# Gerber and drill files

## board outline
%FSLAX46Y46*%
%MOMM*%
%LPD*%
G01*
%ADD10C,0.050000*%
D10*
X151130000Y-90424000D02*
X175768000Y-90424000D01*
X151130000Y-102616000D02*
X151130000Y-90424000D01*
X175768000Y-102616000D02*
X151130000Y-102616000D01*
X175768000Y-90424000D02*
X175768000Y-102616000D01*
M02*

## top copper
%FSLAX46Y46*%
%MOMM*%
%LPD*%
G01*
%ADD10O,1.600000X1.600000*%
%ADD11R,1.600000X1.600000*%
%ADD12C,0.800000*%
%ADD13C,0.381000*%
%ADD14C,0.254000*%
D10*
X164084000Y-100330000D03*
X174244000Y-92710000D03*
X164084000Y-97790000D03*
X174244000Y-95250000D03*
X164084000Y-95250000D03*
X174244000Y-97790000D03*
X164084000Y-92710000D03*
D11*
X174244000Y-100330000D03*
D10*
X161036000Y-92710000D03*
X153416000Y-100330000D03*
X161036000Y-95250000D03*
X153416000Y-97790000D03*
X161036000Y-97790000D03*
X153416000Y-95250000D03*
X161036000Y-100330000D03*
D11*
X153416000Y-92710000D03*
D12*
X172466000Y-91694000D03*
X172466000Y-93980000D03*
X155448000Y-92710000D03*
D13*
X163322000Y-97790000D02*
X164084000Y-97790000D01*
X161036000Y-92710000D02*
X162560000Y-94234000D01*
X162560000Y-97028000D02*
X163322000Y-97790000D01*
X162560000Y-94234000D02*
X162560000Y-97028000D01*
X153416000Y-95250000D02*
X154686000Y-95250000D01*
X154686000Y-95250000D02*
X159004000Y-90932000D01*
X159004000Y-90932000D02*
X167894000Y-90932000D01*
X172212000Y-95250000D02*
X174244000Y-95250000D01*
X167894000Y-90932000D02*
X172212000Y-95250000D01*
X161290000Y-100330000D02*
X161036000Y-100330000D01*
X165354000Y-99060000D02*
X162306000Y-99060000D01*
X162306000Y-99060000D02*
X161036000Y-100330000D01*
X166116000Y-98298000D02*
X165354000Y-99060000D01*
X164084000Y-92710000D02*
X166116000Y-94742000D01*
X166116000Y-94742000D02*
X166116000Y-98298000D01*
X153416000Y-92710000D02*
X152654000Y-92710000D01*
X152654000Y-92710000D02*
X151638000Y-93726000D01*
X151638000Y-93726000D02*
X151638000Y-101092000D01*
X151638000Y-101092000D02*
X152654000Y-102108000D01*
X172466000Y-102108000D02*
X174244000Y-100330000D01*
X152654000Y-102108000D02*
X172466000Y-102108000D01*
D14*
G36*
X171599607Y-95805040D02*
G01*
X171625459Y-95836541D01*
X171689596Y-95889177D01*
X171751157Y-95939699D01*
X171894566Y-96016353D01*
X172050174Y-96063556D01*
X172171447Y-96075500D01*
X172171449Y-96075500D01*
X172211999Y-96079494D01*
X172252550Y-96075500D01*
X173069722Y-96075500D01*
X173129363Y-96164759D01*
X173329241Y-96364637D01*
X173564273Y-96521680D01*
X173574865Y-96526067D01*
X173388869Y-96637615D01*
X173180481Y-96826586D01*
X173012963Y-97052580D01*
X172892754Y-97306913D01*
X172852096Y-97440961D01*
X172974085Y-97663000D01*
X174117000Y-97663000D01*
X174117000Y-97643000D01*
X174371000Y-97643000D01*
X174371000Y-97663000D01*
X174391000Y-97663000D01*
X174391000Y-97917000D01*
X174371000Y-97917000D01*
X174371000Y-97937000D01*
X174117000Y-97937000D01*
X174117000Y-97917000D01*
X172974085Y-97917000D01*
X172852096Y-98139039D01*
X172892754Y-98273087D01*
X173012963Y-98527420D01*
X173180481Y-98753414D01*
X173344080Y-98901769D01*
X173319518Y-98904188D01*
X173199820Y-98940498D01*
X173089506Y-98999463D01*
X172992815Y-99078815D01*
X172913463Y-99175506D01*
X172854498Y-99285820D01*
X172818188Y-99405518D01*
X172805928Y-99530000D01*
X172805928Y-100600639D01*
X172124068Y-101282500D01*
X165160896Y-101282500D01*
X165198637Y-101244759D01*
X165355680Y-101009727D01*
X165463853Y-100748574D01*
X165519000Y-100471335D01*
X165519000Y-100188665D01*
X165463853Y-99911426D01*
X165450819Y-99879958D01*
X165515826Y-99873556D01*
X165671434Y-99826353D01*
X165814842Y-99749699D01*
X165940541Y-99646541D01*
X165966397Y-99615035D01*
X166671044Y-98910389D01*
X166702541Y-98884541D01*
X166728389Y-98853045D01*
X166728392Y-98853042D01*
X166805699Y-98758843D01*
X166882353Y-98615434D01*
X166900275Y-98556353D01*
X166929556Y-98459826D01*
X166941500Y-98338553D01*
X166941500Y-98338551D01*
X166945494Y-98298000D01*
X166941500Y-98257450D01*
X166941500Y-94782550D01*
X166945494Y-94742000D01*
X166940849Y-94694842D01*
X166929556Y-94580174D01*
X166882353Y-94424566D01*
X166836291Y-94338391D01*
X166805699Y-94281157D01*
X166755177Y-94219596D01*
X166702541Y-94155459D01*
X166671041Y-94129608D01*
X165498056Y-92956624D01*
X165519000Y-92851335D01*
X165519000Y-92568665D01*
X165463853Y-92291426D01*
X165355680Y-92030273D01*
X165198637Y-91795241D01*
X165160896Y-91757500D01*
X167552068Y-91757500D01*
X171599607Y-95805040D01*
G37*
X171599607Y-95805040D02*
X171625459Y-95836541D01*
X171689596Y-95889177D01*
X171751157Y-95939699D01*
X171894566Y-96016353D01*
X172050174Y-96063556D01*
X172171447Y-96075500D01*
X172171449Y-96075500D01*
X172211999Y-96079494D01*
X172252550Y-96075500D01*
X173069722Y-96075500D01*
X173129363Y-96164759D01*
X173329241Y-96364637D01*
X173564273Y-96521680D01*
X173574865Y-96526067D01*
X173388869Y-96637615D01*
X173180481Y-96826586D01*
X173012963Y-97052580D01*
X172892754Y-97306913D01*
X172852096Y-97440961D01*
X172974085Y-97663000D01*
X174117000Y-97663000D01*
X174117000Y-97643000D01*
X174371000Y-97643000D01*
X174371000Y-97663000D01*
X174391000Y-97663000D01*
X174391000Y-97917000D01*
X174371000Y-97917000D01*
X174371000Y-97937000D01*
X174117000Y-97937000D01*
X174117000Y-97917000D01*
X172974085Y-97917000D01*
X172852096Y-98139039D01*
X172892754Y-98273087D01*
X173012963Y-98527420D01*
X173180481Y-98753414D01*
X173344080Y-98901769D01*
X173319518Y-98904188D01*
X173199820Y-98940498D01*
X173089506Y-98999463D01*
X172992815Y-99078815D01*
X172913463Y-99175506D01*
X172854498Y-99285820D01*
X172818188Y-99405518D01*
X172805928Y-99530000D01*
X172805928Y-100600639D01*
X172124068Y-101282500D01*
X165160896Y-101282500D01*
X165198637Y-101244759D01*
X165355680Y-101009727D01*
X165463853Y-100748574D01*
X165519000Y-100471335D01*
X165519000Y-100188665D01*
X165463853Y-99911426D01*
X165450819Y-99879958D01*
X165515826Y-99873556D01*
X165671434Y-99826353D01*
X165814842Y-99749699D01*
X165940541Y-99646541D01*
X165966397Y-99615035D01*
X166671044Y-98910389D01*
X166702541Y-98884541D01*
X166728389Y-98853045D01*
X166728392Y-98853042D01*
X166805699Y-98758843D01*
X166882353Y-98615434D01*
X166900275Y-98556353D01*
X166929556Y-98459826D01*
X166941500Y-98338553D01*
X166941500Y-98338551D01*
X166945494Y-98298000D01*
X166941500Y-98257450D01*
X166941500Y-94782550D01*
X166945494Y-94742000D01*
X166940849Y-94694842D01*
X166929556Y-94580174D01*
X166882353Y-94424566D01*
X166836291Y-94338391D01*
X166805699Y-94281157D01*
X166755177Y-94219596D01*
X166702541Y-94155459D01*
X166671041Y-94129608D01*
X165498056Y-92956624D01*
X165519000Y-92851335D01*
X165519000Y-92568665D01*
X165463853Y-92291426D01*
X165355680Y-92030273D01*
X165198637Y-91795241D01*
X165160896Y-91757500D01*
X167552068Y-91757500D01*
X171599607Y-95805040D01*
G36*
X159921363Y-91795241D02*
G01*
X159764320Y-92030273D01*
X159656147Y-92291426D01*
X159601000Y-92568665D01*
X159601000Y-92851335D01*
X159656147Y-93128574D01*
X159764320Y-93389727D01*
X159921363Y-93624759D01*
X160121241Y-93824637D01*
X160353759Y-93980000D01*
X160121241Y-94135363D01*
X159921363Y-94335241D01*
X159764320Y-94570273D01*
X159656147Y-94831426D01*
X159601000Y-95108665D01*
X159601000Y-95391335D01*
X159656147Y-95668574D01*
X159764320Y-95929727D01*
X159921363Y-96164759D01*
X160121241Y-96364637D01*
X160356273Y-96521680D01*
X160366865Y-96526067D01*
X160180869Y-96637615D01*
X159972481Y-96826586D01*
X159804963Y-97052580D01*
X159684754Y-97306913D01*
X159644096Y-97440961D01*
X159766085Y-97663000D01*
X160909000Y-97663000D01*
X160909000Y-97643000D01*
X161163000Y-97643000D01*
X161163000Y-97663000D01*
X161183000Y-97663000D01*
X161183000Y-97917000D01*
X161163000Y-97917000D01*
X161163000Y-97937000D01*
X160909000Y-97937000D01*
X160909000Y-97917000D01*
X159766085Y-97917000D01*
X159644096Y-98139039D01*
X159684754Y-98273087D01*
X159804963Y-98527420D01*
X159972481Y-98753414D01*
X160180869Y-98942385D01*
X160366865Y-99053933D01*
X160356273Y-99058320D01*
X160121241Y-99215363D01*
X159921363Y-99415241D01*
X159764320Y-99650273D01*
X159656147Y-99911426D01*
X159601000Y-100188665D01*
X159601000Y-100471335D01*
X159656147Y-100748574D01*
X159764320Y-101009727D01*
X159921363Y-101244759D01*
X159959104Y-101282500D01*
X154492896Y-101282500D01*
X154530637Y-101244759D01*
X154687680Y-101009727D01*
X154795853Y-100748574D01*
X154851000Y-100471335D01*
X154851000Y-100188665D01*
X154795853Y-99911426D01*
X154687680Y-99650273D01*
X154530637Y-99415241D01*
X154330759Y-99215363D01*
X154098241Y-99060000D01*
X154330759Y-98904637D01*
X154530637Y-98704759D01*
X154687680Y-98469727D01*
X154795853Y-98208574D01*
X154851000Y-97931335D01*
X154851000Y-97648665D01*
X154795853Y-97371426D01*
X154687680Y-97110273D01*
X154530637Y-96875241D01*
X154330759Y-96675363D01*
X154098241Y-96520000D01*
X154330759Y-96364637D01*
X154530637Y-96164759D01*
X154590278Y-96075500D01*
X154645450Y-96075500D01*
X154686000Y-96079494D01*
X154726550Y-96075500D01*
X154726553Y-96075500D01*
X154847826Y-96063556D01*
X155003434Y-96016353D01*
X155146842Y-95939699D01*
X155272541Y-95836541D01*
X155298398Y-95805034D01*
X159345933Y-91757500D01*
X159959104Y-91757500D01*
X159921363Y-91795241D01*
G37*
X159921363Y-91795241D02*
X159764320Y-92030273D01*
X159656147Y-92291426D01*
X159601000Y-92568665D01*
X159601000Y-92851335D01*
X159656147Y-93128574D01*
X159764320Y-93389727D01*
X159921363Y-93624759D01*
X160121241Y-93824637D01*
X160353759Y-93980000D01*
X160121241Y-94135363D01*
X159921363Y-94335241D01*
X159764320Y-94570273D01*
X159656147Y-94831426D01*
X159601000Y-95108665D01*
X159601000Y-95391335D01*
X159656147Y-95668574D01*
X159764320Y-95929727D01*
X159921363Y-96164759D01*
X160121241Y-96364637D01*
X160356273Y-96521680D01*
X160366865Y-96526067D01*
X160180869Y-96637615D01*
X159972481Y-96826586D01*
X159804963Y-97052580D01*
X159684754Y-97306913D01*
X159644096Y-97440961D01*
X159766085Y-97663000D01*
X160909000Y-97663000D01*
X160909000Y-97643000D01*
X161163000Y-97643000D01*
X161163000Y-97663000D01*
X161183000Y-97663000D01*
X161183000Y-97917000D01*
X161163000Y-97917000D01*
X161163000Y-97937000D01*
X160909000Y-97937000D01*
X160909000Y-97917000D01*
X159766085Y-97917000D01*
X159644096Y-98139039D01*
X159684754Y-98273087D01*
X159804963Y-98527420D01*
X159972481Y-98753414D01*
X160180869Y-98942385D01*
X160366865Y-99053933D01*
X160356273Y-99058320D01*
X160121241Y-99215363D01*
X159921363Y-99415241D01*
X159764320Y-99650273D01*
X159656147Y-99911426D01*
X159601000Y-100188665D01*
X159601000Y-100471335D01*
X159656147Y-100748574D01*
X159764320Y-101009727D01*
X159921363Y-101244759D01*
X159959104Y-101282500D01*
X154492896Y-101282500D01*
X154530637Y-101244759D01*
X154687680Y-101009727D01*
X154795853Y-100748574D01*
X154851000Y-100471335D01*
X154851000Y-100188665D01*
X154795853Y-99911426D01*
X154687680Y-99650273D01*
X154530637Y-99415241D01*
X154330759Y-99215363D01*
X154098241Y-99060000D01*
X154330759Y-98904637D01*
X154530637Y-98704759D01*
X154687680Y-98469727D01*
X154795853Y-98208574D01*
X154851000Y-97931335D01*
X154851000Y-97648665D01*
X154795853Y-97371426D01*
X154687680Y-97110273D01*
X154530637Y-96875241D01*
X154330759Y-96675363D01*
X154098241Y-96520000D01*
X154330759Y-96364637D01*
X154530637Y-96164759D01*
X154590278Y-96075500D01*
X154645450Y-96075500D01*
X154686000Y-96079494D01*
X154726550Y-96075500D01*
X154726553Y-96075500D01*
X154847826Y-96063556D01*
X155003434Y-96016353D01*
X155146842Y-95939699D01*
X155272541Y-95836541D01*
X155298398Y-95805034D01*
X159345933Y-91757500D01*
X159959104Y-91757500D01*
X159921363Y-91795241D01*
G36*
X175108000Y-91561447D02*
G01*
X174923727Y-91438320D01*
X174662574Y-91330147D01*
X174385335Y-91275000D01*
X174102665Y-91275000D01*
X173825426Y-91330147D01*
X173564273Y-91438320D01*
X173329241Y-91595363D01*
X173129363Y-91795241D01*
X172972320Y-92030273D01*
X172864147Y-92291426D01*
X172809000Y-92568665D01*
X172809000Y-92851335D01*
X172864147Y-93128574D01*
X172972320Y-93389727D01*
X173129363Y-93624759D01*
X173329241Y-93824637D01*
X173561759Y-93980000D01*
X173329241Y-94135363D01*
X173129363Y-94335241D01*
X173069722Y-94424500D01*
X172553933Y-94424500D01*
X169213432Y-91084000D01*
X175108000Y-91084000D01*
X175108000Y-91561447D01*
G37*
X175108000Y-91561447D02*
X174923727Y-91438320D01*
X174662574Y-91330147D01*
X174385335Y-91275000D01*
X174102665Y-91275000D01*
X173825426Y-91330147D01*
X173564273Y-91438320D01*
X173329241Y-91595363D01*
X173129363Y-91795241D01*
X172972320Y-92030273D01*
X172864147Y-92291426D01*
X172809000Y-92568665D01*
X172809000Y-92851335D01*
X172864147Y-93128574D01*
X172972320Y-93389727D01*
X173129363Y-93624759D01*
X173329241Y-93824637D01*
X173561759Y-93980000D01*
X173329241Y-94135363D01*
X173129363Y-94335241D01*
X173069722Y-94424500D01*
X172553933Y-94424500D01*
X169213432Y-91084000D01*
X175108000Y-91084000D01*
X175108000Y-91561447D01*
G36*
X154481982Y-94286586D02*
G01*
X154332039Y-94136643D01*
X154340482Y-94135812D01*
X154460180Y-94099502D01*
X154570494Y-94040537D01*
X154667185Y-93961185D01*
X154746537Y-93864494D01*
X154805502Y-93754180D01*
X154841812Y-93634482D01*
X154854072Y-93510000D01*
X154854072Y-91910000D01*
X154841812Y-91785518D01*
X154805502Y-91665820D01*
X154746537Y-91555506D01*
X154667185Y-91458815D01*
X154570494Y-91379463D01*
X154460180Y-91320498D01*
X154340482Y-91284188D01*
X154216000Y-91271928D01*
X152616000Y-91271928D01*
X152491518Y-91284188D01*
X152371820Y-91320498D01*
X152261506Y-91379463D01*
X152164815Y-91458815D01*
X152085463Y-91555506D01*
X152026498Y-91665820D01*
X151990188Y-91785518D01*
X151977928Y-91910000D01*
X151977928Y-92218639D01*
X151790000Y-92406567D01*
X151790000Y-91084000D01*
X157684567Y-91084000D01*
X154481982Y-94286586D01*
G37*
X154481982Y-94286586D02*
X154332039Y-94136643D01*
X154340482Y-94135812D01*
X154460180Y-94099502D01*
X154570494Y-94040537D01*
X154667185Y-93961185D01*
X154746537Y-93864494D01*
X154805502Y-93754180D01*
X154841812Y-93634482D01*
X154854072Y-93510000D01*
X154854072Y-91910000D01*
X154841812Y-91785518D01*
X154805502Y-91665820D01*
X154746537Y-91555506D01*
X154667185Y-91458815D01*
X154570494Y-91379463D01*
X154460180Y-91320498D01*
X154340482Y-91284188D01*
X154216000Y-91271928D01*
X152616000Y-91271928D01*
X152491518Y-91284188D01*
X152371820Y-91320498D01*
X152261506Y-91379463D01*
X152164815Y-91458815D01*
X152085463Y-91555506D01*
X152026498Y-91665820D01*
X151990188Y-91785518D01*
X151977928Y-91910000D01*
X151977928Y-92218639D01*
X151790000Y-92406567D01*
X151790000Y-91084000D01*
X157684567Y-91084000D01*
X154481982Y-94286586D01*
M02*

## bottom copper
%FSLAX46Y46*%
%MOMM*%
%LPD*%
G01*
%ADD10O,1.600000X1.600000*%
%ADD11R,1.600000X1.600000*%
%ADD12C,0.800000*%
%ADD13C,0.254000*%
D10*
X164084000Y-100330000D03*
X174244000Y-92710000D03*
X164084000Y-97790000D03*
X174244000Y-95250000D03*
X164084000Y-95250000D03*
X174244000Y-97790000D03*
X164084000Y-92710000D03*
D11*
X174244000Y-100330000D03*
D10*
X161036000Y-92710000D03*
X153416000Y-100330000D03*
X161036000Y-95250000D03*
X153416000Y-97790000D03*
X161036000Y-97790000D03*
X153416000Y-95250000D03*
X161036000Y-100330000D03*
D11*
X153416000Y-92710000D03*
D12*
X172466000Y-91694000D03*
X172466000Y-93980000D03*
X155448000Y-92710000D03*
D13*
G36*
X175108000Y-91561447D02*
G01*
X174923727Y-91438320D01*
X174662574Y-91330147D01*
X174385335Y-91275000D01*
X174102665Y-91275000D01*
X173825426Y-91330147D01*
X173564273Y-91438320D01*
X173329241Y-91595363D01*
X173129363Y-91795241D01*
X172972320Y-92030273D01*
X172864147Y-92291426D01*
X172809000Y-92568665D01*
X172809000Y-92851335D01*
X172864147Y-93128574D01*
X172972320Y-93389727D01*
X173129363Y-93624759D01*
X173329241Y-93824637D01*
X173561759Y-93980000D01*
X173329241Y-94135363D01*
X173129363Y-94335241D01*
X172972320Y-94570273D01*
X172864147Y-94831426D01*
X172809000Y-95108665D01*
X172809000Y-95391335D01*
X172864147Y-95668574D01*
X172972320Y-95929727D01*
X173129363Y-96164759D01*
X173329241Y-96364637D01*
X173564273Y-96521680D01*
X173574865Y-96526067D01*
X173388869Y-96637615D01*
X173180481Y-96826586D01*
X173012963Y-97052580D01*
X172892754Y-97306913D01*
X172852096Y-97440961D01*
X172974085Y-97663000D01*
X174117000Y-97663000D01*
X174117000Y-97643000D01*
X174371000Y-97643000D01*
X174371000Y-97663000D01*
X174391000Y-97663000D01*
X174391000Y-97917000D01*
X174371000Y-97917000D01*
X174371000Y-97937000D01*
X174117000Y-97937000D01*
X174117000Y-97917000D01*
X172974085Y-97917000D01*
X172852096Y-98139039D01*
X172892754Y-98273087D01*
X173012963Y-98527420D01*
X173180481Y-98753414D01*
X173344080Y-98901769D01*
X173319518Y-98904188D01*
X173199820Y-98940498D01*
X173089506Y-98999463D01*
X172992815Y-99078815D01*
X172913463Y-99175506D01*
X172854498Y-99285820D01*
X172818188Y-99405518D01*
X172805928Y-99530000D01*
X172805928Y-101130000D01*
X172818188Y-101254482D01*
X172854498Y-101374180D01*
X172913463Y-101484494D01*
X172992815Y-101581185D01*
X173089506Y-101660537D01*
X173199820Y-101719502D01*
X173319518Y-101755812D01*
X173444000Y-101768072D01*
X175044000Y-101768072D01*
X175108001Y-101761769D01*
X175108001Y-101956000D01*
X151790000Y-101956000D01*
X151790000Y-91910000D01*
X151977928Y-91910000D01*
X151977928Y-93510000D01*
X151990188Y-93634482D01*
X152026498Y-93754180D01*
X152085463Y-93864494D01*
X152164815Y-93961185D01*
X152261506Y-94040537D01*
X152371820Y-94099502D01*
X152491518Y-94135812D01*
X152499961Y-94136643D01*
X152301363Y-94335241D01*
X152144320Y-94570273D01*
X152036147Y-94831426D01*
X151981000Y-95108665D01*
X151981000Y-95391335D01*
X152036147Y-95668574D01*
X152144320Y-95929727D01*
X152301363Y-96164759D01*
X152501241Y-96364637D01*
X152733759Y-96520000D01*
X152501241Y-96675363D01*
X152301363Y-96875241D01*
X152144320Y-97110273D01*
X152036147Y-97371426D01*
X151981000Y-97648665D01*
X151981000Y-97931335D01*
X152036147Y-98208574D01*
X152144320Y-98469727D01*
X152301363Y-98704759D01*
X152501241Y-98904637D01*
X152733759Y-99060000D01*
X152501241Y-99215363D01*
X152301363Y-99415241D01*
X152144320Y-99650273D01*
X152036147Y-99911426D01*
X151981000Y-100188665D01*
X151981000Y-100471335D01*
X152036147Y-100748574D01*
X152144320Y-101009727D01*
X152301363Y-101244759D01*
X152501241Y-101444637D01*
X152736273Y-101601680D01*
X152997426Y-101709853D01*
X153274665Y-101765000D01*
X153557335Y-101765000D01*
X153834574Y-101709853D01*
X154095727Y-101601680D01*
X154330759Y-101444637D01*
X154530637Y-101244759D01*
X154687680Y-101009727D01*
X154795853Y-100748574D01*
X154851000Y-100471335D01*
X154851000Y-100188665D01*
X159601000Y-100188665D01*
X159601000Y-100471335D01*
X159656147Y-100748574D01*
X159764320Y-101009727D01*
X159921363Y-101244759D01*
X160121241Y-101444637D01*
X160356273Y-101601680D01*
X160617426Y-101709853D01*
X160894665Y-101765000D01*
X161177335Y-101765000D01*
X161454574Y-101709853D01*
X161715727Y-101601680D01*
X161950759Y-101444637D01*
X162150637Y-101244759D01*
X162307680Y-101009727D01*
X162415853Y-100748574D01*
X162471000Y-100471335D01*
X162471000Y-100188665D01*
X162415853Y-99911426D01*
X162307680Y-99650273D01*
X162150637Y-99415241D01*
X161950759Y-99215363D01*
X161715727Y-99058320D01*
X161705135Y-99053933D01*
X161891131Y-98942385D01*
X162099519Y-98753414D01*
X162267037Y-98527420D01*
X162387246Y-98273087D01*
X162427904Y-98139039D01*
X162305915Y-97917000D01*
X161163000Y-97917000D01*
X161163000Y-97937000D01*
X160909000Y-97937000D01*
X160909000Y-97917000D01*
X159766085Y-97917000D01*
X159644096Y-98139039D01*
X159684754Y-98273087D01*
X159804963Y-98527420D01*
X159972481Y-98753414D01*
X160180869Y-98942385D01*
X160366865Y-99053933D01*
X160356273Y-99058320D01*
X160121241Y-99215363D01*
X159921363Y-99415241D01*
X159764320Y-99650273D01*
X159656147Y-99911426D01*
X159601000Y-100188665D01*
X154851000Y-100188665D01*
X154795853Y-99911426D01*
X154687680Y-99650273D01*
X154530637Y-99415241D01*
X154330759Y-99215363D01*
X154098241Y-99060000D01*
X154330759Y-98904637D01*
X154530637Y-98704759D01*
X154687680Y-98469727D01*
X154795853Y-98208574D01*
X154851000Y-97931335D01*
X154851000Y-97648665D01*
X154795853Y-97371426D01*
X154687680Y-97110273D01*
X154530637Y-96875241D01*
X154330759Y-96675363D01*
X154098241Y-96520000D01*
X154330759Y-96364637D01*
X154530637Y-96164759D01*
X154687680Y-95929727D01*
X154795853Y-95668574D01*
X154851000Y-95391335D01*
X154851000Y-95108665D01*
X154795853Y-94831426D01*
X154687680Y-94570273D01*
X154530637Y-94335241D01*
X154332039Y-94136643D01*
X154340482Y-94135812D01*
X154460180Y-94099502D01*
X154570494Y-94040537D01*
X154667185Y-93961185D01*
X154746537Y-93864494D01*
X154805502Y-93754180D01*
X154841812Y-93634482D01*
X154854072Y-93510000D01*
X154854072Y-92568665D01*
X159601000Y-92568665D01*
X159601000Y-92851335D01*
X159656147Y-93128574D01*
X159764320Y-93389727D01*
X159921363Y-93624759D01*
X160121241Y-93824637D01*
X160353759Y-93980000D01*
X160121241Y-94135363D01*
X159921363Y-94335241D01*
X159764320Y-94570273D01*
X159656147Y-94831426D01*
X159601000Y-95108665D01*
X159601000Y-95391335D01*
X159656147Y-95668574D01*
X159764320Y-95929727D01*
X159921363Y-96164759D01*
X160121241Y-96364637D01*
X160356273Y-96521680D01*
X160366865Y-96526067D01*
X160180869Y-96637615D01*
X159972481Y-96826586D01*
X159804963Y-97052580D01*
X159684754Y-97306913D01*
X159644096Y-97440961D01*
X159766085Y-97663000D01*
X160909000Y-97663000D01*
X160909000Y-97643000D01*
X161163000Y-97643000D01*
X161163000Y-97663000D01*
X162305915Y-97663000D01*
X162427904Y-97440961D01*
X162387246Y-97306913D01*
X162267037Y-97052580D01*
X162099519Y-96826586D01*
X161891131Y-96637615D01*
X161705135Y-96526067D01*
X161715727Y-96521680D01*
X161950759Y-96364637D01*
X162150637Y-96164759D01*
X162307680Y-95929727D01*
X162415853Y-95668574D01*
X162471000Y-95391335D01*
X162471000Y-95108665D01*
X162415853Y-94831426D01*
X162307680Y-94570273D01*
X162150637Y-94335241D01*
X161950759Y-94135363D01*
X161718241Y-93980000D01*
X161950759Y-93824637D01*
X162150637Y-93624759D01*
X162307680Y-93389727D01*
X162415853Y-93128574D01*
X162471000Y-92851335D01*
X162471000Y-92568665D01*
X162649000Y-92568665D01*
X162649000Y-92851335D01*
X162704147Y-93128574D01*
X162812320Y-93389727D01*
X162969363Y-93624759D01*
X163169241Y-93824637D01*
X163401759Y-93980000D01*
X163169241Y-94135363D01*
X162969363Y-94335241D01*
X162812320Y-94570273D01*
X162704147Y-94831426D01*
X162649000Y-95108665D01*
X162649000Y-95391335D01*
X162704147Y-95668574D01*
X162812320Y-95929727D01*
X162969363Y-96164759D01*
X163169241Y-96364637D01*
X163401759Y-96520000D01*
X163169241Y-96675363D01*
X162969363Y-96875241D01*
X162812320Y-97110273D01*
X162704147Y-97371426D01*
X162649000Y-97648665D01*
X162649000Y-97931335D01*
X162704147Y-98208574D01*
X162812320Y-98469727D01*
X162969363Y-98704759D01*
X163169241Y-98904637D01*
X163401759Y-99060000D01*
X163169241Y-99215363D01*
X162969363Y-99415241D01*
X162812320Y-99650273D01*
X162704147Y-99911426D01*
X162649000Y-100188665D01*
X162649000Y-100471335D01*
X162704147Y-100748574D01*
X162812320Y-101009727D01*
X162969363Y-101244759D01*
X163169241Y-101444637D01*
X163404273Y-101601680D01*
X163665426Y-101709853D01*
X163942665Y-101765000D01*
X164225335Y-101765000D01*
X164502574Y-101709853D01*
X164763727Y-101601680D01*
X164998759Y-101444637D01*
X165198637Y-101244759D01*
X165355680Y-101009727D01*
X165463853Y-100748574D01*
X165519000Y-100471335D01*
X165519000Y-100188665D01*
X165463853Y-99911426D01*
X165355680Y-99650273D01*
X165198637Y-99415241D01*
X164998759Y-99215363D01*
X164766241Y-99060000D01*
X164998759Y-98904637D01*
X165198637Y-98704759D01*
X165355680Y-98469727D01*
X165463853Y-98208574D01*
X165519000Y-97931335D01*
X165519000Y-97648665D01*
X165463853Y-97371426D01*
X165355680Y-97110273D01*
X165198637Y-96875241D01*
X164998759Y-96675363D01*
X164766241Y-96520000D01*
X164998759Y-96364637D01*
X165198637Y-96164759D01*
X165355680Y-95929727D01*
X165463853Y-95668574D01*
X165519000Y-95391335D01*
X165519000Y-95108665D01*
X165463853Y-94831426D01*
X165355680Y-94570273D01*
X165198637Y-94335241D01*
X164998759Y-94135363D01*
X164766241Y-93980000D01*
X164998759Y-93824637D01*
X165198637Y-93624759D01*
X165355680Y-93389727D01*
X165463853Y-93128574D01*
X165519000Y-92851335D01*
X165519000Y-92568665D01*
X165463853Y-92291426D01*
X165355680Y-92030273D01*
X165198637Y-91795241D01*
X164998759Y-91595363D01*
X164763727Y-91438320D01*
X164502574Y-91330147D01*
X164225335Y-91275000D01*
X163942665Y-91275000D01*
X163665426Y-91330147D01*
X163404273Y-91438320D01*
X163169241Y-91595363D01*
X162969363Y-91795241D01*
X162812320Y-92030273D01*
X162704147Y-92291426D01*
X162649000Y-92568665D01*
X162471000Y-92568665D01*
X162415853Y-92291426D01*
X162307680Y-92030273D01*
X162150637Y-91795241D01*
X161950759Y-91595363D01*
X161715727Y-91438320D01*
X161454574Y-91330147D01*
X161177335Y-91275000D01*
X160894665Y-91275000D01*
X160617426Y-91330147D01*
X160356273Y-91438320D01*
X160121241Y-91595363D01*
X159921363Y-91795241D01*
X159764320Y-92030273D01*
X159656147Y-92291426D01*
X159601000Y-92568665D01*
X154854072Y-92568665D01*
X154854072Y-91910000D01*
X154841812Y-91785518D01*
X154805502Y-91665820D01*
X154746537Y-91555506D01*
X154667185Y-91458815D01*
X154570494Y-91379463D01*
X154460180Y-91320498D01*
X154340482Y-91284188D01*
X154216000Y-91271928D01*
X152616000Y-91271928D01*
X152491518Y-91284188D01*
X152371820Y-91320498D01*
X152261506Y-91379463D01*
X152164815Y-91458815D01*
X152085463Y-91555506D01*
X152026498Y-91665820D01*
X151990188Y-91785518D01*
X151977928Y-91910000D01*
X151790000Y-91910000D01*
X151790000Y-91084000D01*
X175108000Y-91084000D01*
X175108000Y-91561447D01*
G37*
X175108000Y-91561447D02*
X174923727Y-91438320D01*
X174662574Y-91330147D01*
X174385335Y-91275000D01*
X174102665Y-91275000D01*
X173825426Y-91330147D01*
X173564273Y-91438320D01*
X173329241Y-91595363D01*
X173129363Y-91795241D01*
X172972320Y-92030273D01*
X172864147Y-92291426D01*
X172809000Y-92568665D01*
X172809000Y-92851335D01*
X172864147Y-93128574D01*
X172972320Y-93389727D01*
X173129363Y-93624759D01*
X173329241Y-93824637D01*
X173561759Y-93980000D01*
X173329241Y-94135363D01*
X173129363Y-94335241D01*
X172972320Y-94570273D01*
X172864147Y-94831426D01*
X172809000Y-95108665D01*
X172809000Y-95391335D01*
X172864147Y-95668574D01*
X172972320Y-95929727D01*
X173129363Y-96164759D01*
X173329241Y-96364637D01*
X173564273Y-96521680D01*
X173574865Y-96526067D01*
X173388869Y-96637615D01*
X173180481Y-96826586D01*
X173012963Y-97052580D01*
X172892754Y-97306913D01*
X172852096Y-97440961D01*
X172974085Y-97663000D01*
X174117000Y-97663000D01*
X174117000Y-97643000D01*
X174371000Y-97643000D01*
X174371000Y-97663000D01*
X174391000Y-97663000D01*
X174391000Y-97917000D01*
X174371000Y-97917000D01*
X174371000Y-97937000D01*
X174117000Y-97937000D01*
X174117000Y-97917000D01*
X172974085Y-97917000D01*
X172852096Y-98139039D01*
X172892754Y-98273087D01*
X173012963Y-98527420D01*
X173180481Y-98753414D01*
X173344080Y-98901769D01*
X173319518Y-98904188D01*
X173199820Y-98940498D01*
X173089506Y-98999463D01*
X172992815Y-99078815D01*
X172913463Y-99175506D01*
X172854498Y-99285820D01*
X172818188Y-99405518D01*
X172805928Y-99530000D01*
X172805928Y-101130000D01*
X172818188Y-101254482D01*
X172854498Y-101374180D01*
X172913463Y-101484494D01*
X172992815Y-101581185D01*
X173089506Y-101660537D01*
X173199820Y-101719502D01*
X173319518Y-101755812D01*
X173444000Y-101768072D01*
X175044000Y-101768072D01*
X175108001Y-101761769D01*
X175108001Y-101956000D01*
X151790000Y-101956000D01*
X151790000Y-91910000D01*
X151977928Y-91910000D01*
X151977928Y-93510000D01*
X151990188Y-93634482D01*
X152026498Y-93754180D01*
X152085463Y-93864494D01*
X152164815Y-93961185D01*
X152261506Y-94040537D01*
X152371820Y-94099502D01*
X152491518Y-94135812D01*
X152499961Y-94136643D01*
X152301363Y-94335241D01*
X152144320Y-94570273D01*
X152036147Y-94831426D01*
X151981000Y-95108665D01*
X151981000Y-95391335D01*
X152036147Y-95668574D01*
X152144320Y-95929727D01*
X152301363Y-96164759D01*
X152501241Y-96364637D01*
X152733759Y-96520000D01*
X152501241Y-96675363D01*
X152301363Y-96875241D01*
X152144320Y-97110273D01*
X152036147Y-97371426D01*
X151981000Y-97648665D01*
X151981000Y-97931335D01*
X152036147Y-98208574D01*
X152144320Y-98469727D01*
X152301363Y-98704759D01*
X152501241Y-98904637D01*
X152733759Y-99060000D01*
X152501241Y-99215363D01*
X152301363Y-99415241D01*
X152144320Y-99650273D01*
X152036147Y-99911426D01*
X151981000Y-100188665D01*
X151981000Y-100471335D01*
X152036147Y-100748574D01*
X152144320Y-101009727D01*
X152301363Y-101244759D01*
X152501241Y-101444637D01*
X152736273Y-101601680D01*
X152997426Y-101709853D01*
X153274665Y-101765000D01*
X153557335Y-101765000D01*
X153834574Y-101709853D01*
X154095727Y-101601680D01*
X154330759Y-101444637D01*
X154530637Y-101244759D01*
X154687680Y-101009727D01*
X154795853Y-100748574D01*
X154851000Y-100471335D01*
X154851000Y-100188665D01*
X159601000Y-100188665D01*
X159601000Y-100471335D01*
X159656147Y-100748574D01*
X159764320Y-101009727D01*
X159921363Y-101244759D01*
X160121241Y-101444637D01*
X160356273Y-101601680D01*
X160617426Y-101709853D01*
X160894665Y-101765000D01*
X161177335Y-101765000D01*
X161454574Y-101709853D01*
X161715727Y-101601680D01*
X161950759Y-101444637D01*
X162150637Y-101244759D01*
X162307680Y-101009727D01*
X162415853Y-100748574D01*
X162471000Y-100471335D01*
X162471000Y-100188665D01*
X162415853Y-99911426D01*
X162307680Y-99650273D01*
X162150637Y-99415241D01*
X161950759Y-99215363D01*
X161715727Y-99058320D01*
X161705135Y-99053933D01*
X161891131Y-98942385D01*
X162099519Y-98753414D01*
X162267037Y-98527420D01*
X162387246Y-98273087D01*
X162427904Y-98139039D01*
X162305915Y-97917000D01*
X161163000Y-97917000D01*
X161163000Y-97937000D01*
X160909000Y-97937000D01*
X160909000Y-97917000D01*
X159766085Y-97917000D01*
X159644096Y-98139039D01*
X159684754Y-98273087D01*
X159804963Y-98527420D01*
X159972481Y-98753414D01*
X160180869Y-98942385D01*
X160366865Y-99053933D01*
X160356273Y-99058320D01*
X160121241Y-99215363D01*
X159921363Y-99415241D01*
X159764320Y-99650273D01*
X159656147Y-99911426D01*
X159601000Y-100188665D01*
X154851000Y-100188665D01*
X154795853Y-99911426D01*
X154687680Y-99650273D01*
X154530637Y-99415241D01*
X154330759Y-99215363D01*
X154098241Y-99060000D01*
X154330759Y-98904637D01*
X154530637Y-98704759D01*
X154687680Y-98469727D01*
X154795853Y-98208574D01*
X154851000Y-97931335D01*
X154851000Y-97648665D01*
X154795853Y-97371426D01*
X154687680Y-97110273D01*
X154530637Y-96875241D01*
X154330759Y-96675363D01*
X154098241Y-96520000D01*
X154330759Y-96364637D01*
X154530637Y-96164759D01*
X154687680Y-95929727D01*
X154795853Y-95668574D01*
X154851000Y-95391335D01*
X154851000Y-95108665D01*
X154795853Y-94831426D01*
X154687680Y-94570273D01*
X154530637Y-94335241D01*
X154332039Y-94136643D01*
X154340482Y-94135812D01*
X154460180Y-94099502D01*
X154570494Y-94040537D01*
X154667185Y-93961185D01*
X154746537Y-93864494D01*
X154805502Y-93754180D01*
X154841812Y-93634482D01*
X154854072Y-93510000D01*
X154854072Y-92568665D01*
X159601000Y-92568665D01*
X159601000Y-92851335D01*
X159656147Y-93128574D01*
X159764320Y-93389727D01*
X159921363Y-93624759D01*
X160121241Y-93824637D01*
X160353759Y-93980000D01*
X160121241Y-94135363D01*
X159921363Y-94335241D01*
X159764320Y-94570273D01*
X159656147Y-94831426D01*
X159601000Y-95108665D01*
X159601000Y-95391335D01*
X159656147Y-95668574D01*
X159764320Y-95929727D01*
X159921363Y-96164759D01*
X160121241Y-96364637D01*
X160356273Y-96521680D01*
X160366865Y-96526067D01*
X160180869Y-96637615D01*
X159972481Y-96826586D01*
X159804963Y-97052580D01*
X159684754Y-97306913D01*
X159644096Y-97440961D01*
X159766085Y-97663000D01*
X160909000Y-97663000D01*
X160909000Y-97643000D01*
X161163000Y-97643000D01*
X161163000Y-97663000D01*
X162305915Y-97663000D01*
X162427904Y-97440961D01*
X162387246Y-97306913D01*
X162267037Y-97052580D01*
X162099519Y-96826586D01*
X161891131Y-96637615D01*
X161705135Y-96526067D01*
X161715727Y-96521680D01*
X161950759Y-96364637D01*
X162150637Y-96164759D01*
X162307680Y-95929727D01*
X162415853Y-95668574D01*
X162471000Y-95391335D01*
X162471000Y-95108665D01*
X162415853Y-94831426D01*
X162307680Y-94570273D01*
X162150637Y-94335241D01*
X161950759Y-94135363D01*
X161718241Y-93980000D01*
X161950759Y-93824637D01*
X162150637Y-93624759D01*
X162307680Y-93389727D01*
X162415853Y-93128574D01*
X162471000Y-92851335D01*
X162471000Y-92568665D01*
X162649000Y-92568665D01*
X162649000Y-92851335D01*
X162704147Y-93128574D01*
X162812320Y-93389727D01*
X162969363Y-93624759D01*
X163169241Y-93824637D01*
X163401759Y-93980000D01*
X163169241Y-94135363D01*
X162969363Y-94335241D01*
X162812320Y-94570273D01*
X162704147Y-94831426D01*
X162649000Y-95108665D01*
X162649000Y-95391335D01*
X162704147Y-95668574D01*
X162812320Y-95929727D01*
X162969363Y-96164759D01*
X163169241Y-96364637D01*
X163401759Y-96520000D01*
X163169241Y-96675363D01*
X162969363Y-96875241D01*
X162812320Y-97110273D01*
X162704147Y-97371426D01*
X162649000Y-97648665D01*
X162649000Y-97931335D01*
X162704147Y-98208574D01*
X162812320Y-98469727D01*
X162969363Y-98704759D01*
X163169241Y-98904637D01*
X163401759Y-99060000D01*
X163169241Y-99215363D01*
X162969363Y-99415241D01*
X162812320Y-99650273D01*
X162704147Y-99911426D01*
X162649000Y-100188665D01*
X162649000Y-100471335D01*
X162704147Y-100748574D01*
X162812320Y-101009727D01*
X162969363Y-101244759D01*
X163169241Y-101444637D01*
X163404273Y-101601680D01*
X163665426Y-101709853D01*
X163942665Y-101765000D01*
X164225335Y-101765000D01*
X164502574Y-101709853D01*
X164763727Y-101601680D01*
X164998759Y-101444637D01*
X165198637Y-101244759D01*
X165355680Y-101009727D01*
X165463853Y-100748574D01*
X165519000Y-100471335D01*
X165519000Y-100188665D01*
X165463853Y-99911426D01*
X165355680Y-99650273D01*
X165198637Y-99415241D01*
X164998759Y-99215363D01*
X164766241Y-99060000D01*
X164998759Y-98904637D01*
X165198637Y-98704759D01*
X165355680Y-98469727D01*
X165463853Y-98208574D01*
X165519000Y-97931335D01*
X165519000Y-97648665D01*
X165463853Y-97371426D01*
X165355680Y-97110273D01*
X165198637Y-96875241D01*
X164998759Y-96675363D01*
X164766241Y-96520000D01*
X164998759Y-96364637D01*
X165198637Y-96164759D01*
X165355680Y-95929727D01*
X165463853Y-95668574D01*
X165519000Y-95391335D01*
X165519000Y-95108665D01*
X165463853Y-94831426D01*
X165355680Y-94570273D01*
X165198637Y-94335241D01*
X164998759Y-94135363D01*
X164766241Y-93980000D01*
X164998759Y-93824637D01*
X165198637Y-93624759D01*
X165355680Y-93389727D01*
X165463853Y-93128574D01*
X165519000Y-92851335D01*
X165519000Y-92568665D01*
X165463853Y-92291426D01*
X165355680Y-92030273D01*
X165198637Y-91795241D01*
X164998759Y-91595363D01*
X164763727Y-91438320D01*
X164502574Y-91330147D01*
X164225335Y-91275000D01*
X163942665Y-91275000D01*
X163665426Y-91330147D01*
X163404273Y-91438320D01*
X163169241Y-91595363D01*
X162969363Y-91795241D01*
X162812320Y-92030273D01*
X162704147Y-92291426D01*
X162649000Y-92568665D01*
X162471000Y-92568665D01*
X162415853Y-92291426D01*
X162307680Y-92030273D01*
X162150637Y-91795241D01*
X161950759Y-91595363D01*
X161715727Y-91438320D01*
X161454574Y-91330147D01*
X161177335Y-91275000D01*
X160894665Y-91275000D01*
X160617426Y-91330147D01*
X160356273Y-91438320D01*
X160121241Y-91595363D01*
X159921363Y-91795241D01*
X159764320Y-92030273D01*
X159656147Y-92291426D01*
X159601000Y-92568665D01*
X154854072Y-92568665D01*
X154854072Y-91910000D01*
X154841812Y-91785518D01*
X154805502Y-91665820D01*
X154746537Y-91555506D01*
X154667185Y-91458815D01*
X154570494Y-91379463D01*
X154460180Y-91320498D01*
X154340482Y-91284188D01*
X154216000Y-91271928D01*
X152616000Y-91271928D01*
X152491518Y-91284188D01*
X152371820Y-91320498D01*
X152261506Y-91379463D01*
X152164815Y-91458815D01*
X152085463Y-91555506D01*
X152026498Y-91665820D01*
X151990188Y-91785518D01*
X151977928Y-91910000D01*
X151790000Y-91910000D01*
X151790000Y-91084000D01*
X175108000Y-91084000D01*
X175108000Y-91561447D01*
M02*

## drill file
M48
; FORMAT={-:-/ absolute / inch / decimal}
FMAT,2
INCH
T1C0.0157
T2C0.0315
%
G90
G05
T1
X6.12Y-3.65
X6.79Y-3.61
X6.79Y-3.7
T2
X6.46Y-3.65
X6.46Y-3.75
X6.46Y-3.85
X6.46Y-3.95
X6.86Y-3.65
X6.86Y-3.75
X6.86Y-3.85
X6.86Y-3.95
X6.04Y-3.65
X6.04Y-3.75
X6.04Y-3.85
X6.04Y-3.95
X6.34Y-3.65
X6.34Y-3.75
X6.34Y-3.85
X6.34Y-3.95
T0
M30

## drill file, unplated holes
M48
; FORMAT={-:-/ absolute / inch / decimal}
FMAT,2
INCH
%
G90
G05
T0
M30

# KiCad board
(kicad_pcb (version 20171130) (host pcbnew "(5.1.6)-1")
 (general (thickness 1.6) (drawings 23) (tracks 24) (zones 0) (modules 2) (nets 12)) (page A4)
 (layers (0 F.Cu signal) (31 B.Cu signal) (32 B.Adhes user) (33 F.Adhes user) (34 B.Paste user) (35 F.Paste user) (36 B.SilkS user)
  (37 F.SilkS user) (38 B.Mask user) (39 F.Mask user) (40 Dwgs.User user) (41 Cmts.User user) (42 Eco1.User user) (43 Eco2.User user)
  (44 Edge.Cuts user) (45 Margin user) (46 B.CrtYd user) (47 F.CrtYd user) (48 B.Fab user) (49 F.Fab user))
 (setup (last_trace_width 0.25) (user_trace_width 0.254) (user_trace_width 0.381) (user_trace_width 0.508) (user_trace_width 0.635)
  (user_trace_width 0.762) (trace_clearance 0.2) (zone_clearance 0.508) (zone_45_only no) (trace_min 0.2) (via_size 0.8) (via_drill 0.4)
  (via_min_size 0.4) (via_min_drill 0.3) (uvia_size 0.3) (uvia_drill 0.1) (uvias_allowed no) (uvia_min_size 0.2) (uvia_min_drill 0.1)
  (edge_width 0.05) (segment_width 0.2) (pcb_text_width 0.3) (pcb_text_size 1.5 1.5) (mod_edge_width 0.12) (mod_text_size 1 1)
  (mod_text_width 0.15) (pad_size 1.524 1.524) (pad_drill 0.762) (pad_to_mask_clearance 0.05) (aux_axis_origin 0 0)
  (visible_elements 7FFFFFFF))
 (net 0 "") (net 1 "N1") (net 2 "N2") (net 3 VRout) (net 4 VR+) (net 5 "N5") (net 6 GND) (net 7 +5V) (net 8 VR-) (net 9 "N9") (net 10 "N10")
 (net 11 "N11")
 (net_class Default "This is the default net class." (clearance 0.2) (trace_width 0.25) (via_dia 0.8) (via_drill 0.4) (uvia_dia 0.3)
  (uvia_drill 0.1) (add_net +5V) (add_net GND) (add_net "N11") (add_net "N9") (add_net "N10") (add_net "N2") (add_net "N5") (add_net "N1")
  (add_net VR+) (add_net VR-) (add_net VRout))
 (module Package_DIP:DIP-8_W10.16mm (layer F.Cu) (at 174.244 100.33 180)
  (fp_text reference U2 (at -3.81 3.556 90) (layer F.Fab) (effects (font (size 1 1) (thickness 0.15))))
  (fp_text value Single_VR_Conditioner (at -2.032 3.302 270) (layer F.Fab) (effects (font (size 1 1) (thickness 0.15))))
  (pad 8 thru_hole oval (at 10.16 0 180) (size 1.6 1.6) (drill 0.8) (layers *.Cu *.Mask) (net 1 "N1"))
  (pad 4 thru_hole oval (at 0 7.62 180) (size 1.6 1.6) (drill 0.8) (layers *.Cu *.Mask) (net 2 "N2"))
  (pad 7 thru_hole oval (at 10.16 2.54 180) (size 1.6 1.6) (drill 0.8) (layers *.Cu *.Mask) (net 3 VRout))
  (pad 3 thru_hole oval (at 0 5.08 180) (size 1.6 1.6) (drill 0.8) (layers *.Cu *.Mask) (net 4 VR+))
  (pad 6 thru_hole oval (at 10.16 5.08 180) (size 1.6 1.6) (drill 0.8) (layers *.Cu *.Mask) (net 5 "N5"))
  (pad 2 thru_hole oval (at 0 2.54 180) (size 1.6 1.6) (drill 0.8) (layers *.Cu *.Mask) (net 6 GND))
  (pad 5 thru_hole oval (at 10.16 7.62 180) (size 1.6 1.6) (drill 0.8) (layers *.Cu *.Mask) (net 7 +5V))
  (pad 1 thru_hole rect (at 0 0 180) (size 1.6 1.6) (drill 0.8) (layers *.Cu *.Mask) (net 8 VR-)))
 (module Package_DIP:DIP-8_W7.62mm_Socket (layer F.Cu) (at 153.416 92.71)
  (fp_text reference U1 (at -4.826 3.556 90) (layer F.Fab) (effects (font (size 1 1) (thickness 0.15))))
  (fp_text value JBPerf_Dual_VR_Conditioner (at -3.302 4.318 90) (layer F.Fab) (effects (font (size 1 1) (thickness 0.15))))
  (pad 8 thru_hole oval (at 7.62 0) (size 1.6 1.6) (drill 0.8) (layers *.Cu *.Mask) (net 3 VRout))
  (pad 4 thru_hole oval (at 0 7.62) (size 1.6 1.6) (drill 0.8) (layers *.Cu *.Mask) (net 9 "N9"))
  (pad 7 thru_hole oval (at 7.62 2.54) (size 1.6 1.6) (drill 0.8) (layers *.Cu *.Mask) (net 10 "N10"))
  (pad 3 thru_hole oval (at 0 5.08) (size 1.6 1.6) (drill 0.8) (layers *.Cu *.Mask) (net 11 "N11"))
  (pad 6 thru_hole oval (at 7.62 5.08) (size 1.6 1.6) (drill 0.8) (layers *.Cu *.Mask) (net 6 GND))
  (pad 2 thru_hole oval (at 0 2.54) (size 1.6 1.6) (drill 0.8) (layers *.Cu *.Mask) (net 4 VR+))
  (pad 5 thru_hole oval (at 7.62 7.62) (size 1.6 1.6) (drill 0.8) (layers *.Cu *.Mask) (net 7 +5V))
  (pad 1 thru_hole rect (at 0 0) (size 1.6 1.6) (drill 0.8) (layers *.Cu *.Mask) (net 8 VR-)))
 (gr_line (start 151.13 90.424) (end 175.768 90.424) (layer Edge.Cuts) (width 0.05))
 (gr_line (start 151.13 102.616) (end 151.13 90.424) (layer Edge.Cuts) (width 0.05))
 (gr_line (start 175.768 102.616) (end 151.13 102.616) (layer Edge.Cuts) (width 0.05))
 (gr_line (start 175.768 90.424) (end 175.768 102.616) (layer Edge.Cuts) (width 0.05))
 (segment (start 163.322 97.79) (end 164.084 97.79) (width 0.381) (layer F.Cu) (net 3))
 (segment (start 161.036 92.71) (end 162.56 94.234) (width 0.381) (layer F.Cu) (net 3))
 (segment (start 162.56 97.028) (end 163.322 97.79) (width 0.381) (layer F.Cu) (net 3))
 (segment (start 162.56 94.234) (end 162.56 97.028) (width 0.381) (layer F.Cu) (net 3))
 (via (at 172.466 91.694) (size 0.8) (drill 0.4) (layers F.Cu B.Cu) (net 6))
 (via (at 172.466 93.98) (size 0.8) (drill 0.4) (layers F.Cu B.Cu) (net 6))
 (via (at 155.448 92.71) (size 0.8) (drill 0.4) (layers F.Cu B.Cu) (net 6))
 (segment (start 153.416 95.25) (end 154.686 95.25) (width 0.381) (layer F.Cu) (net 4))
 (segment (start 154.686 95.25) (end 159.004 90.932) (width 0.381) (layer F.Cu) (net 4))
 (segment (start 159.004 90.932) (end 167.894 90.932) (width 0.381) (layer F.Cu) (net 4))
 (segment (start 172.212 95.25) (end 174.244 95.25) (width 0.381) (layer F.Cu) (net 4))
 (segment (start 167.894 90.932) (end 172.212 95.25) (width 0.381) (layer F.Cu) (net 4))
 (segment (start 161.29 100.33) (end 161.036 100.33) (width 0.381) (layer F.Cu) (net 7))
 (segment (start 165.354 99.06) (end 162.306 99.06) (width 0.381) (layer F.Cu) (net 7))
 (segment (start 162.306 99.06) (end 161.036 100.33) (width 0.381) (layer F.Cu) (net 7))
 (segment (start 166.116 98.298) (end 165.354 99.06) (width 0.381) (layer F.Cu) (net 7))
 (segment (start 164.084 92.71) (end 166.116 94.742) (width 0.381) (layer F.Cu) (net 7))
 (segment (start 166.116 94.742) (end 166.116 98.298) (width 0.381) (layer F.Cu) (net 7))
 (segment (start 153.416 92.71) (end 152.654 92.71) (width 0.381) (layer F.Cu) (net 8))
 (segment (start 152.654 92.71) (end 151.638 93.726) (width 0.381) (layer F.Cu) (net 8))
 (segment (start 151.638 93.726) (end 151.638 101.092) (width 0.381) (layer F.Cu) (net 8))
 (segment (start 151.638 101.092) (end 152.654 102.108) (width 0.381) (layer F.Cu) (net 8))
 (segment (start 172.466 102.108) (end 174.244 100.33) (width 0.381) (layer F.Cu) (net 8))
 (segment (start 152.654 102.108) (end 172.466 102.108) (width 0.381) (layer F.Cu) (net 8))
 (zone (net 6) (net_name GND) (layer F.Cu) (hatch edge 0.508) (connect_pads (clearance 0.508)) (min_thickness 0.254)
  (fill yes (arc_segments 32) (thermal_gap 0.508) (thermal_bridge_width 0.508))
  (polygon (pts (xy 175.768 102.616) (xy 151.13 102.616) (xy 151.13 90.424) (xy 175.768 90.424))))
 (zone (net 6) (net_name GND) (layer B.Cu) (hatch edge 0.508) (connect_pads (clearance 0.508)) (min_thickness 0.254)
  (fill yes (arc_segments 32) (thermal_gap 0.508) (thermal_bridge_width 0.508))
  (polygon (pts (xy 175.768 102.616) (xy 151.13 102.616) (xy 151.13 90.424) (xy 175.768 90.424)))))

